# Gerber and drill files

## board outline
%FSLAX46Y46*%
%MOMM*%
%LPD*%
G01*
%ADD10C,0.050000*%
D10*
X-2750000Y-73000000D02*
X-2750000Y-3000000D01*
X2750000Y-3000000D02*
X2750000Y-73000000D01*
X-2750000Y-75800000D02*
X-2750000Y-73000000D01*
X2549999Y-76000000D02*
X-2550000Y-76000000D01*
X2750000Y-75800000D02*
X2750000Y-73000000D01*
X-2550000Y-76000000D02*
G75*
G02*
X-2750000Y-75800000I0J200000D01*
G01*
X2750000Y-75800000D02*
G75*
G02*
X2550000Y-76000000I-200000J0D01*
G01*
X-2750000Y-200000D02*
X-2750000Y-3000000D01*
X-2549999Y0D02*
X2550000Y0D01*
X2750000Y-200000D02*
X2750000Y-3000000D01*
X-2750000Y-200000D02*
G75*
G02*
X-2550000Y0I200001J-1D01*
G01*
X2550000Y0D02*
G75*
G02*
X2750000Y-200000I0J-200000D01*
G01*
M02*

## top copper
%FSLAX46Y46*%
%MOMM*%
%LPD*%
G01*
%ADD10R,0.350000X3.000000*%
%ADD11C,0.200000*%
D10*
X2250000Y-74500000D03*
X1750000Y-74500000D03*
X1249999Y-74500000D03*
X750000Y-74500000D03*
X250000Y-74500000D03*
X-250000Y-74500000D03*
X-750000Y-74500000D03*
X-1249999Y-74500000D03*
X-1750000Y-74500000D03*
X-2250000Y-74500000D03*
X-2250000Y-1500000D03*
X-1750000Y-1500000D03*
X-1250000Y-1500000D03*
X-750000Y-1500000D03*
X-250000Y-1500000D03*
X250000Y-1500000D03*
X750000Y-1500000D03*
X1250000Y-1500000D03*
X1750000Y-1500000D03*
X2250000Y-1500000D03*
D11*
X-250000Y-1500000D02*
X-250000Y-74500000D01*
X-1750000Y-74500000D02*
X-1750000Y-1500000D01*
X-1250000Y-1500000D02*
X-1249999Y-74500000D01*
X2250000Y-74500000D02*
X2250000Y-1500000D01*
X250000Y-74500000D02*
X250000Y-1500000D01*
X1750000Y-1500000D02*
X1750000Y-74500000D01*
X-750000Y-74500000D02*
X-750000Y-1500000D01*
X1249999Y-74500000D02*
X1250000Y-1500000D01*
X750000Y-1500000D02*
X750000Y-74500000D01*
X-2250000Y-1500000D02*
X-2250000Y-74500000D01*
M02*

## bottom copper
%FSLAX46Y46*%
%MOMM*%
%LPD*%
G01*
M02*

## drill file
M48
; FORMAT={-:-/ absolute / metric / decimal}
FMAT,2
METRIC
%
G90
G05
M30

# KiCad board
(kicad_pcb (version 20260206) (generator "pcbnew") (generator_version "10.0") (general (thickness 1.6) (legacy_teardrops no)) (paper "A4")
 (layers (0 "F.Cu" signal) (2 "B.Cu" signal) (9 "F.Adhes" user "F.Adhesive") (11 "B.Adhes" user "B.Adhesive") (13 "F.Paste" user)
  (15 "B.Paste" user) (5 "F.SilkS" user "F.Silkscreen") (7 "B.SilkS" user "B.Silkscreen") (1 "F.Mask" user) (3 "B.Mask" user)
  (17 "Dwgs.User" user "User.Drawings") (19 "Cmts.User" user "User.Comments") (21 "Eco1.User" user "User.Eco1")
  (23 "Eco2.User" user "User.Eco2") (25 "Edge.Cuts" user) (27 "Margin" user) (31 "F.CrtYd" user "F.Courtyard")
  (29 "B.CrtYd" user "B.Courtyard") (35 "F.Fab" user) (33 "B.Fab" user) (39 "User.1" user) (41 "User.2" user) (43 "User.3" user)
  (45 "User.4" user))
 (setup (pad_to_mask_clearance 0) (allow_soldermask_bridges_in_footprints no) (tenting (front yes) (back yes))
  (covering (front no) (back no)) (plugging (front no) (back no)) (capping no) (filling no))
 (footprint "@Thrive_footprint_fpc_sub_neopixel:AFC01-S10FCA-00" (layer "F.Cu") (at 0 74.5 180)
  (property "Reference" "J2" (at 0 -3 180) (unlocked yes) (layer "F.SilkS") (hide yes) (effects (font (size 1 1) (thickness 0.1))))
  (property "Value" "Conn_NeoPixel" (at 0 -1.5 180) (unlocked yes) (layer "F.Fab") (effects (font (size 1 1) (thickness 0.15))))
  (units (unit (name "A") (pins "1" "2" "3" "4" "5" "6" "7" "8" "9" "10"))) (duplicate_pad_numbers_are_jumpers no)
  (fp_line (start 2.75 -1.3) (end 2.75 1.5) (stroke (width 0.05) (type default)) (layer "Edge.Cuts"))
  (fp_line (start -2.549999 -1.5) (end 2.55 -1.5) (stroke (width 0.05) (type default)) (layer "Edge.Cuts"))
  (fp_line (start -2.75 -1.3) (end -2.75 1.5) (stroke (width 0.05) (type default)) (layer "Edge.Cuts"))
  (fp_arc (start 2.55 -1.5) (mid 2.691421 -1.441422) (end 2.75 -1.3) (stroke (width 0.05) (type default)) (layer "Edge.Cuts"))
  (fp_arc (start -2.75 -1.3) (mid -2.691421 -1.441422) (end -2.55 -1.5) (stroke (width 0.05) (type default)) (layer "Edge.Cuts"))
  (pad "1" smd rect (at -2.25 0 180) (size 0.35 3) (layers "F.Cu" "F.Mask" "F.Paste") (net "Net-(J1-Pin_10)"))
  (pad "2" smd rect (at -1.75 0 180) (size 0.35 3) (layers "F.Cu" "F.Mask" "F.Paste") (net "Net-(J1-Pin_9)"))
  (pad "3" smd rect (at -1.249999 0 180) (size 0.35 3) (layers "F.Cu" "F.Mask" "F.Paste") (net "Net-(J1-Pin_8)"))
  (pad "4" smd rect (at -0.75 0 180) (size 0.35 3) (layers "F.Cu" "F.Mask" "F.Paste") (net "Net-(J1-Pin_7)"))
  (pad "5" smd rect (at -0.25 0 180) (size 0.35 3) (layers "F.Cu" "F.Mask" "F.Paste") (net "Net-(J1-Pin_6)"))
  (pad "6" smd rect (at 0.25 0 180) (size 0.35 3) (layers "F.Cu" "F.Mask" "F.Paste") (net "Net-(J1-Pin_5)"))
  (pad "7" smd rect (at 0.75 0 180) (size 0.35 3) (layers "F.Cu" "F.Mask" "F.Paste") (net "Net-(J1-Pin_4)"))
  (pad "8" smd rect (at 1.249999 0 180) (size 0.35 3) (layers "F.Cu" "F.Mask" "F.Paste") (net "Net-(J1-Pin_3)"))
  (pad "9" smd rect (at 1.75 0 180) (size 0.35 3) (layers "F.Cu" "F.Mask" "F.Paste") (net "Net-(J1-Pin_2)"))
  (pad "10" smd rect (at 2.25 0 180) (size 0.35 3) (layers "F.Cu" "F.Mask" "F.Paste") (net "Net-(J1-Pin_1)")))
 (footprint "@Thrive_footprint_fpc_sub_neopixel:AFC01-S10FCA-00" (layer "F.Cu") (at 0 1.5)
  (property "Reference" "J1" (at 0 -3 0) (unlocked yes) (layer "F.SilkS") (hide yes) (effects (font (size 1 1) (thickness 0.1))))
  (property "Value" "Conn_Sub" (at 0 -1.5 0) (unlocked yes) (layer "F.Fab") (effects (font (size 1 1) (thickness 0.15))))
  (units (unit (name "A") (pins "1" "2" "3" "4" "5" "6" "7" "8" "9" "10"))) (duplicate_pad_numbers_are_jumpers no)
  (fp_line (start -2.75 -1.3) (end -2.75 1.5) (stroke (width 0.05) (type default)) (layer "Edge.Cuts"))
  (fp_line (start -2.549999 -1.5) (end 2.55 -1.5) (stroke (width 0.05) (type default)) (layer "Edge.Cuts"))
  (fp_line (start 2.75 -1.3) (end 2.75 1.5) (stroke (width 0.05) (type default)) (layer "Edge.Cuts"))
  (fp_arc (start -2.75 -1.3) (mid -2.691421 -1.441421) (end -2.55 -1.5) (stroke (width 0.05) (type default)) (layer "Edge.Cuts"))
  (fp_arc (start 2.55 -1.5) (mid 2.691421 -1.441421) (end 2.75 -1.3) (stroke (width 0.05) (type default)) (layer "Edge.Cuts"))
  (pad "1" smd rect (at -2.25 0) (size 0.35 3) (layers "F.Cu" "F.Mask" "F.Paste") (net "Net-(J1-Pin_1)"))
  (pad "2" smd rect (at -1.75 0) (size 0.35 3) (layers "F.Cu" "F.Mask" "F.Paste") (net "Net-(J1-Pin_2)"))
  (pad "3" smd rect (at -1.25 0) (size 0.35 3) (layers "F.Cu" "F.Mask" "F.Paste") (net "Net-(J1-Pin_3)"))
  (pad "4" smd rect (at -0.75 0) (size 0.35 3) (layers "F.Cu" "F.Mask" "F.Paste") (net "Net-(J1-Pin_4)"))
  (pad "5" smd rect (at -0.25 0) (size 0.35 3) (layers "F.Cu" "F.Mask" "F.Paste") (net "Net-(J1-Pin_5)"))
  (pad "6" smd rect (at 0.25 0) (size 0.35 3) (layers "F.Cu" "F.Mask" "F.Paste") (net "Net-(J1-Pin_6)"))
  (pad "7" smd rect (at 0.75 0) (size 0.35 3) (layers "F.Cu" "F.Mask" "F.Paste") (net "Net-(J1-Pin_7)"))
  (pad "8" smd rect (at 1.25 0) (size 0.35 3) (layers "F.Cu" "F.Mask" "F.Paste") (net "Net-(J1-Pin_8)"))
  (pad "9" smd rect (at 1.75 0) (size 0.35 3) (layers "F.Cu" "F.Mask" "F.Paste") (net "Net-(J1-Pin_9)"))
  (pad "10" smd rect (at 2.25 0) (size 0.35 3) (layers "F.Cu" "F.Mask" "F.Paste") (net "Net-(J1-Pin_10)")))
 (gr_line (start -2.75 73) (end -2.75 3) (stroke (width 0.05) (type default)) (layer "Edge.Cuts"))
 (gr_line (start 2.75 3) (end 2.75 73) (stroke (width 0.05) (type default)) (layer "Edge.Cuts"))
 (segment (start -0.25 1.5) (end -0.25 74.5) (width 0.2) (layer "F.Cu") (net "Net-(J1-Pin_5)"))
 (segment (start -1.75 74.5) (end -1.75 1.5) (width 0.2) (layer "F.Cu") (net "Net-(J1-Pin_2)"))
 (segment (start -1.25 1.5) (end -1.249999 74.5) (width 0.2) (layer "F.Cu") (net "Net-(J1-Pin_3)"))
 (segment (start 2.25 74.5) (end 2.25 1.5) (width 0.2) (layer "F.Cu") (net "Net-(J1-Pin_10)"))
 (segment (start 0.25 74.5) (end 0.25 1.5) (width 0.2) (layer "F.Cu") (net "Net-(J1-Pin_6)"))
 (segment (start 1.75 1.5) (end 1.75 74.5) (width 0.2) (layer "F.Cu") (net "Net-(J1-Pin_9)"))
 (segment (start -0.75 74.5) (end -0.75 1.5) (width 0.2) (layer "F.Cu") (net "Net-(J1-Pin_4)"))
 (segment (start 1.249999 74.5) (end 1.25 1.5) (width 0.2) (layer "F.Cu") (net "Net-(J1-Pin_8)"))
 (segment (start 0.75 1.5) (end 0.75 74.5) (width 0.2) (layer "F.Cu") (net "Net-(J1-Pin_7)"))
 (segment (start -2.25 1.5) (end -2.25 74.5) (width 0.2) (layer "F.Cu") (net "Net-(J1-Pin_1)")))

